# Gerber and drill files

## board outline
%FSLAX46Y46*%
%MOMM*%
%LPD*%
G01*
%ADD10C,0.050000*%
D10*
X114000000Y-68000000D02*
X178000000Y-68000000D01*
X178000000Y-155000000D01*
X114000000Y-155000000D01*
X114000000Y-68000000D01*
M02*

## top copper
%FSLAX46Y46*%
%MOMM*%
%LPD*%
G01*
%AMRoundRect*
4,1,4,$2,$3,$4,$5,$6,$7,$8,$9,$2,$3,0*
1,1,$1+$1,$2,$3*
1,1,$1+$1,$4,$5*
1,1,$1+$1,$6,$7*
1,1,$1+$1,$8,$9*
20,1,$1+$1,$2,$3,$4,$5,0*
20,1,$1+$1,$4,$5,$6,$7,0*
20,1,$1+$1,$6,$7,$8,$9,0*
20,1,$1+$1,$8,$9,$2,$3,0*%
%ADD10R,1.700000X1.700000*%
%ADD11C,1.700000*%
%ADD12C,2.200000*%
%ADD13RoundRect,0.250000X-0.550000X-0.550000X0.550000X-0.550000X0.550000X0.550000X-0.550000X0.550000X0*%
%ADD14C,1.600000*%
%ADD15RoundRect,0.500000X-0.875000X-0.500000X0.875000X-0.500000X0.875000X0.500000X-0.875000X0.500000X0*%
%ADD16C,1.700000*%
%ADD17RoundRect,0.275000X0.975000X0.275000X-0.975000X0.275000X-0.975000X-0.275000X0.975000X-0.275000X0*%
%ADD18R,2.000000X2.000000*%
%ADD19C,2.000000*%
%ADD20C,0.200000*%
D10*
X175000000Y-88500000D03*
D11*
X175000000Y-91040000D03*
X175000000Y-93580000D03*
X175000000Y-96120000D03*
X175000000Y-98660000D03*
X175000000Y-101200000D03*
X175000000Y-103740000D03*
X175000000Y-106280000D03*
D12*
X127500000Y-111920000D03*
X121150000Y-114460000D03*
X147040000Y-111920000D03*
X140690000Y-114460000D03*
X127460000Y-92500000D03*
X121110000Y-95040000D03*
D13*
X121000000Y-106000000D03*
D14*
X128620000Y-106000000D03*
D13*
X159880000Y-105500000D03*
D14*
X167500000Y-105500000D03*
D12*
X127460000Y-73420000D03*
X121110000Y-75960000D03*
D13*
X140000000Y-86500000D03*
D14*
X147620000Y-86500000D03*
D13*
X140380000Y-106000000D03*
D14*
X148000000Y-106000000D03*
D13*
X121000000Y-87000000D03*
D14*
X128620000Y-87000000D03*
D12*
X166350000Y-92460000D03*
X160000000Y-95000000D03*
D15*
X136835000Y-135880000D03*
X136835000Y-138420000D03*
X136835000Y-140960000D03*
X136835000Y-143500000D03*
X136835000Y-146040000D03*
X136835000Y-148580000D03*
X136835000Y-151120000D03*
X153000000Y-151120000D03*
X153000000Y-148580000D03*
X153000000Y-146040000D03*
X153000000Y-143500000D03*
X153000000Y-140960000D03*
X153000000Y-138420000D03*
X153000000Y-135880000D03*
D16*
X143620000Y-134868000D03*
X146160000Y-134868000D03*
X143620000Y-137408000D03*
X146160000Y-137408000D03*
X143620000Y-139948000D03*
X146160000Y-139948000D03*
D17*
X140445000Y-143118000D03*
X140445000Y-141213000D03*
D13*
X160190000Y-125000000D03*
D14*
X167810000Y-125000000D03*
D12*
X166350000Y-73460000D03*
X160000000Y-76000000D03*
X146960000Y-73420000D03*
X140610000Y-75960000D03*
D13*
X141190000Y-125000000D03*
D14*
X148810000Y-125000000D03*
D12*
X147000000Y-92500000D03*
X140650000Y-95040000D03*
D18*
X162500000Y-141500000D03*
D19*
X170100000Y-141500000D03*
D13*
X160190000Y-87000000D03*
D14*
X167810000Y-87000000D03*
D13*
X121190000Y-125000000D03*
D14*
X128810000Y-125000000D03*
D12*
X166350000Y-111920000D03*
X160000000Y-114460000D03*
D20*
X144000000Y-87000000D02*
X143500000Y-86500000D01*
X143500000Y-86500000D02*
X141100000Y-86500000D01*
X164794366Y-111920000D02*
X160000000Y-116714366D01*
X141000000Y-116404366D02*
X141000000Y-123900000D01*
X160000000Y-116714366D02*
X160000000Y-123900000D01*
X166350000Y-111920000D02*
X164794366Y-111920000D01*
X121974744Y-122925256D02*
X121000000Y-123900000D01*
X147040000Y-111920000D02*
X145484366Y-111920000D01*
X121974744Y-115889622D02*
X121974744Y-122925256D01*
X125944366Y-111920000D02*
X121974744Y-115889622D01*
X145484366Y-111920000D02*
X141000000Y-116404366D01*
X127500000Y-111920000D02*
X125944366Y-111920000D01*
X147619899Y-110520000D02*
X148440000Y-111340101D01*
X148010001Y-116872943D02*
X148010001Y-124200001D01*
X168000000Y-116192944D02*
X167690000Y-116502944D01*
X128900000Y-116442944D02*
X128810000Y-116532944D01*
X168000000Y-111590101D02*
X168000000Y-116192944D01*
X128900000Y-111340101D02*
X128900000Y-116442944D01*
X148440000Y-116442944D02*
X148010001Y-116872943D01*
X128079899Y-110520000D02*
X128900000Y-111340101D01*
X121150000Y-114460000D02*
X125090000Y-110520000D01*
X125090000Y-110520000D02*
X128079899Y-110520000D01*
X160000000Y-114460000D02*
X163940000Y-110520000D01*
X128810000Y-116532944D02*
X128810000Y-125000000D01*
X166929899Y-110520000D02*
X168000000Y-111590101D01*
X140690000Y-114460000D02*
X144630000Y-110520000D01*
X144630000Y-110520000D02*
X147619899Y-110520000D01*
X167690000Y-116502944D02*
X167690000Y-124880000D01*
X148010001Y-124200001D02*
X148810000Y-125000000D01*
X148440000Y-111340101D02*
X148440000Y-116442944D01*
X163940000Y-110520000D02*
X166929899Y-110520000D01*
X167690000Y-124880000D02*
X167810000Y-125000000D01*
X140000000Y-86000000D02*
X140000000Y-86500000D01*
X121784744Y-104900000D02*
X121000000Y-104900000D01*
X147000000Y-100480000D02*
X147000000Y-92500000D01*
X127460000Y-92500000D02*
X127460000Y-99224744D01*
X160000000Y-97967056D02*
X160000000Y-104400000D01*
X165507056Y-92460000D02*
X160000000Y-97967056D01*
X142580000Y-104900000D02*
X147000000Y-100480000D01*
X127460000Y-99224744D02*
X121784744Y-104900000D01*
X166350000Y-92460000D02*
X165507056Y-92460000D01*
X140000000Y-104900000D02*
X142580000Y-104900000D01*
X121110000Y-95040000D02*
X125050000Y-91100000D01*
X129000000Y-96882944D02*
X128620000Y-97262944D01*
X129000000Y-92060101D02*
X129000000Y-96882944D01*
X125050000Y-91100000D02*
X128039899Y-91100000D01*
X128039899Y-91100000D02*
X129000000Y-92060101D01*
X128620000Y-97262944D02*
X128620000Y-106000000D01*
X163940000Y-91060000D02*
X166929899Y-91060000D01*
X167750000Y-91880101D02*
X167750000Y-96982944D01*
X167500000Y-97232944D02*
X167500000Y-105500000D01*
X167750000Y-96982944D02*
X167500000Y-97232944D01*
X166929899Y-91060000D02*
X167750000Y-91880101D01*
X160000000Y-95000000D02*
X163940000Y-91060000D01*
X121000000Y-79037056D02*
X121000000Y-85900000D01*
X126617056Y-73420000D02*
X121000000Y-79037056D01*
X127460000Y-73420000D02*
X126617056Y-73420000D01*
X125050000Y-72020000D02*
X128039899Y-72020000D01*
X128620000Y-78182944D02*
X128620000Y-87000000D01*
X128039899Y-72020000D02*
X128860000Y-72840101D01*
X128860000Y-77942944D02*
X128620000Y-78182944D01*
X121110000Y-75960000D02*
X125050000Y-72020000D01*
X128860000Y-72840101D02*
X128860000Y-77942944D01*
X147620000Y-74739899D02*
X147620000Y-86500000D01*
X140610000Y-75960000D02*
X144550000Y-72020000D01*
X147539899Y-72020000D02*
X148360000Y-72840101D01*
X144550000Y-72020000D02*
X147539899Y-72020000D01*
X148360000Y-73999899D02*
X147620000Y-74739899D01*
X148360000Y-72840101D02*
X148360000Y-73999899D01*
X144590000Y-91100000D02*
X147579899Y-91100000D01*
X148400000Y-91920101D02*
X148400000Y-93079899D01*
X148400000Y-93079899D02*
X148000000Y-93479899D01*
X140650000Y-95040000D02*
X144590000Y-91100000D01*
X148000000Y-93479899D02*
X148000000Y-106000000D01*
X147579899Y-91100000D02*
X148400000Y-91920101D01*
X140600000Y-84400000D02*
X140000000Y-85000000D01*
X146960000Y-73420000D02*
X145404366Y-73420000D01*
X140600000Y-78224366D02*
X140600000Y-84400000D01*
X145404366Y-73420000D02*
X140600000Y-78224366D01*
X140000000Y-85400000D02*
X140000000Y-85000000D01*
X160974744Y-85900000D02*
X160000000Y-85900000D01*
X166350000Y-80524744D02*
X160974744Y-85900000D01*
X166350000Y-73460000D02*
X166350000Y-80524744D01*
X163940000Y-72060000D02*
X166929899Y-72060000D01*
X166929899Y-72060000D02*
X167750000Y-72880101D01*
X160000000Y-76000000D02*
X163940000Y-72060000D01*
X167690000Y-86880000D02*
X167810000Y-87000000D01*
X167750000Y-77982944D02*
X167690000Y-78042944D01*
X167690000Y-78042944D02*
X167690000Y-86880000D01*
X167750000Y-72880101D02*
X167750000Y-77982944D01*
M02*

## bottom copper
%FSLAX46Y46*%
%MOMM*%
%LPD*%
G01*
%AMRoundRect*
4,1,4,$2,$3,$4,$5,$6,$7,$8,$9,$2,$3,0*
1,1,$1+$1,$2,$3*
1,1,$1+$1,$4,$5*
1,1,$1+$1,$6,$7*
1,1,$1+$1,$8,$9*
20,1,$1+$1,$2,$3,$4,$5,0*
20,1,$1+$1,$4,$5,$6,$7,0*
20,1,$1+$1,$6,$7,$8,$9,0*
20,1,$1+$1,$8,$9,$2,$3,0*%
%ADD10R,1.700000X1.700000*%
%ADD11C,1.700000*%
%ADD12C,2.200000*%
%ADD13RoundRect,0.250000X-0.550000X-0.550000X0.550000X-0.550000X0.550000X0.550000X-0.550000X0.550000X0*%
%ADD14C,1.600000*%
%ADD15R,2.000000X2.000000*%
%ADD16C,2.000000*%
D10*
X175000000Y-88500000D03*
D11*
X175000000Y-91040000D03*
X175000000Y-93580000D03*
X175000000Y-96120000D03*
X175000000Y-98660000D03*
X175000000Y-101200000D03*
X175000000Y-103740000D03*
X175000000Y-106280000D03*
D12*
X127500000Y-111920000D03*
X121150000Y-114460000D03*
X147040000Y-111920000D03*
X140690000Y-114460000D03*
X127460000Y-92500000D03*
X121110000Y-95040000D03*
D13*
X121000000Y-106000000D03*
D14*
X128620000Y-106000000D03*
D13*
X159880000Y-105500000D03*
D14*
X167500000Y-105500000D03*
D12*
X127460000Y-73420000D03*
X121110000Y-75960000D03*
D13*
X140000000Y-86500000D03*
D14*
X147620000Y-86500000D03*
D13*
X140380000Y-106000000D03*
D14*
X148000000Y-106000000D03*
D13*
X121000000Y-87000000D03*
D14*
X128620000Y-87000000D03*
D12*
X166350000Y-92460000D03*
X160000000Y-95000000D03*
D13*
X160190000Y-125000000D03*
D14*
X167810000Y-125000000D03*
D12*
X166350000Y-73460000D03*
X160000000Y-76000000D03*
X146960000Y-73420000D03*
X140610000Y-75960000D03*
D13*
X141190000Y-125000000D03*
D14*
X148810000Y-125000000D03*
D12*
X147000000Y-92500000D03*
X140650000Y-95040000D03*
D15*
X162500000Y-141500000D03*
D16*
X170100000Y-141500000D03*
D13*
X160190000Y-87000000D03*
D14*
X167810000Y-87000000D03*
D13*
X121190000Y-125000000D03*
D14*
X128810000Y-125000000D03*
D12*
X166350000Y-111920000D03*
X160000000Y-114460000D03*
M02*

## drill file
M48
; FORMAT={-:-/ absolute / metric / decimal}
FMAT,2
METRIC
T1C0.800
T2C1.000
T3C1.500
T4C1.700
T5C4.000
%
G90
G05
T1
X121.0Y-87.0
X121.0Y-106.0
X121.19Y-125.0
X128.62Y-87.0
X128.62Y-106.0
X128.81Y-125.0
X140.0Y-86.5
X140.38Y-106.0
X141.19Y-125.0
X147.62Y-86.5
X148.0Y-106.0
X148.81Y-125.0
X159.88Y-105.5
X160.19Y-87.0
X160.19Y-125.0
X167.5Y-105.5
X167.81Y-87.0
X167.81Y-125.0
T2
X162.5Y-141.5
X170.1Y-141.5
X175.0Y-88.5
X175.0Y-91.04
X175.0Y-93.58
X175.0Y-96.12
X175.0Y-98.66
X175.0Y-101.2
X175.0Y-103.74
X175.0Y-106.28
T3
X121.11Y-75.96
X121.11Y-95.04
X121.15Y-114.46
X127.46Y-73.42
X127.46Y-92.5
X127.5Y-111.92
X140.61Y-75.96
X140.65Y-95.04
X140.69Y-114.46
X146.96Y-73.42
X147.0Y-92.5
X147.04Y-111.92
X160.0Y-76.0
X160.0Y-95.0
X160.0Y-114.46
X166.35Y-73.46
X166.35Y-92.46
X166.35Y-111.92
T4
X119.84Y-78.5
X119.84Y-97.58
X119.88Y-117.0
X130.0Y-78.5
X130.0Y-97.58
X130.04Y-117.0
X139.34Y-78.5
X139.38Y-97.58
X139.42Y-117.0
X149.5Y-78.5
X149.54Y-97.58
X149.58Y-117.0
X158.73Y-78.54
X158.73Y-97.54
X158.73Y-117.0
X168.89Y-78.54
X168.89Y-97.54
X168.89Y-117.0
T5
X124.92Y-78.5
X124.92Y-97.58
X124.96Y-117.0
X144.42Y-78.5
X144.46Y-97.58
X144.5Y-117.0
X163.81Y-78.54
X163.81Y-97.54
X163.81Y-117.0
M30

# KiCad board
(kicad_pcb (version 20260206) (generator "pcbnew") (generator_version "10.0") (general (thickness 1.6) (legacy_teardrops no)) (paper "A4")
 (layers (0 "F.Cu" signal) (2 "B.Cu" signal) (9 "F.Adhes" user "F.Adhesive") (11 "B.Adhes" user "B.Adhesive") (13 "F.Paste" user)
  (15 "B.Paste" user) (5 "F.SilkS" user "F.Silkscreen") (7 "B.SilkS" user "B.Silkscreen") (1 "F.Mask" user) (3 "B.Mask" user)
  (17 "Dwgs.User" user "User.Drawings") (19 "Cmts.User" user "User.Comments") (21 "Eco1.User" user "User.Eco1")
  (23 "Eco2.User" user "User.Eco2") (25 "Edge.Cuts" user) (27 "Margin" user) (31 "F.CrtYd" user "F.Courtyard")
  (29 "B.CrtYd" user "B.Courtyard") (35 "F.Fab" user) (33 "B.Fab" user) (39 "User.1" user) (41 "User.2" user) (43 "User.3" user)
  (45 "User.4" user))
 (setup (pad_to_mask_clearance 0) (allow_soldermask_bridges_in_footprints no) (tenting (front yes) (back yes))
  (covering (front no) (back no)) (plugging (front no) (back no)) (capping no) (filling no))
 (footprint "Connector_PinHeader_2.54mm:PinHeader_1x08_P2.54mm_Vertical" (layer "F.Cu") (at 175 88.5)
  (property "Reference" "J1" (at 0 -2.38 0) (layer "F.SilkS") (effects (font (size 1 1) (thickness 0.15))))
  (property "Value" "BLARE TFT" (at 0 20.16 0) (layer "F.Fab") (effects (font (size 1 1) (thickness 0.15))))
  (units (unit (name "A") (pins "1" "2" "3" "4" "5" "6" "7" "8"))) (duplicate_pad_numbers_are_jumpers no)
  (pad "1" thru_hole rect (at 0 0) (size 1.7 1.7) (drill 1) (layers "*.Cu" "*.Mask") (remove_unused_layers no) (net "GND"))
  (pad "2" thru_hole circle (at 0 2.54) (size 1.7 1.7) (drill 1) (layers "*.Cu" "*.Mask") (remove_unused_layers no) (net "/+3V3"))
  (pad "3" thru_hole circle (at 0 5.08) (size 1.7 1.7) (drill 1) (layers "*.Cu" "*.Mask") (remove_unused_layers no) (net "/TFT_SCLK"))
  (pad "4" thru_hole circle (at 0 7.62) (size 1.7 1.7) (drill 1) (layers "*.Cu" "*.Mask") (remove_unused_layers no) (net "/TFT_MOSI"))
  (pad "5" thru_hole circle (at 0 10.16) (size 1.7 1.7) (drill 1) (layers "*.Cu" "*.Mask") (remove_unused_layers no) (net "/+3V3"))
  (pad "6" thru_hole circle (at 0 12.7) (size 1.7 1.7) (drill 1) (layers "*.Cu" "*.Mask") (remove_unused_layers no) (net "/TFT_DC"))
  (pad "7" thru_hole circle (at 0 15.24) (size 1.7 1.7) (drill 1) (layers "*.Cu" "*.Mask") (remove_unused_layers no) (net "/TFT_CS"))
  (pad "8" thru_hole circle (at 0 17.78) (size 1.7 1.7) (drill 1) (layers "*.Cu" "*.Mask") (remove_unused_layers no) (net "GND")))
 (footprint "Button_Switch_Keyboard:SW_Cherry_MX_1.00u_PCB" (layer "F.Cu") (at 127.5 111.92)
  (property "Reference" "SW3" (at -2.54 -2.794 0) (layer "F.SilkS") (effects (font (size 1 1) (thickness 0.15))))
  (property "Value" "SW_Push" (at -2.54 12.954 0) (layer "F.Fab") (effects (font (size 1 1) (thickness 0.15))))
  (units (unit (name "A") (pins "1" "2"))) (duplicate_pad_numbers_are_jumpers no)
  (pad "" np_thru_hole circle (at -7.62 5.08) (size 1.7 1.7) (drill 1.7) (layers "*.Cu" "*.Mask"))
  (pad "" np_thru_hole circle (at -2.54 5.08) (size 4 4) (drill 4) (layers "*.Cu" "*.Mask"))
  (pad "" np_thru_hole circle (at 2.54 5.08) (size 1.7 1.7) (drill 1.7) (layers "*.Cu" "*.Mask"))
  (pad "1" thru_hole circle (at 0 0) (size 2.2 2.2) (drill 1.5) (layers "*.Cu" "*.Mask") (remove_unused_layers no) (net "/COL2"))
  (pad "2" thru_hole circle (at -6.35 2.54) (size 2.2 2.2) (drill 1.5) (layers "*.Cu" "*.Mask") (remove_unused_layers no) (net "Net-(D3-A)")))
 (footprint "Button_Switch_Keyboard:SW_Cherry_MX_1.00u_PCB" (layer "F.Cu") (at 147.04 111.92)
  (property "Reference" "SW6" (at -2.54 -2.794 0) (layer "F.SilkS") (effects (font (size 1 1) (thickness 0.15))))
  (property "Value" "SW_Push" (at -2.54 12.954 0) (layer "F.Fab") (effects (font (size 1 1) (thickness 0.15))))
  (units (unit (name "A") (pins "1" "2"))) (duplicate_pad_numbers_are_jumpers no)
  (pad "" np_thru_hole circle (at -7.62 5.08) (size 1.7 1.7) (drill 1.7) (layers "*.Cu" "*.Mask"))
  (pad "" np_thru_hole circle (at -2.54 5.08) (size 4 4) (drill 4) (layers "*.Cu" "*.Mask"))
  (pad "" np_thru_hole circle (at 2.54 5.08) (size 1.7 1.7) (drill 1.7) (layers "*.Cu" "*.Mask"))
  (pad "1" thru_hole circle (at 0 0) (size 2.2 2.2) (drill 1.5) (layers "*.Cu" "*.Mask") (remove_unused_layers no) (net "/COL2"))
  (pad "2" thru_hole circle (at -6.35 2.54) (size 2.2 2.2) (drill 1.5) (layers "*.Cu" "*.Mask") (remove_unused_layers no) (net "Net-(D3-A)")))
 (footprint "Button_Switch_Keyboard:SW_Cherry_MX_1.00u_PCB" (layer "F.Cu") (at 127.46 92.5)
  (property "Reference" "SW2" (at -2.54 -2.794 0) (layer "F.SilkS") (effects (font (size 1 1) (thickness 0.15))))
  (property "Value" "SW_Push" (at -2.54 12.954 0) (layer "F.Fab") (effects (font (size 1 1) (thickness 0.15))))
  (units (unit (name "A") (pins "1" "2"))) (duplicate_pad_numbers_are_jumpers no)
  (pad "" np_thru_hole circle (at -7.62 5.08) (size 1.7 1.7) (drill 1.7) (layers "*.Cu" "*.Mask"))
  (pad "" np_thru_hole circle (at -2.54 5.08) (size 4 4) (drill 4) (layers "*.Cu" "*.Mask"))
  (pad "" np_thru_hole circle (at 2.54 5.08) (size 1.7 1.7) (drill 1.7) (layers "*.Cu" "*.Mask"))
  (pad "1" thru_hole circle (at 0 0) (size 2.2 2.2) (drill 1.5) (layers "*.Cu" "*.Mask") (remove_unused_layers no) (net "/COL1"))
  (pad "2" thru_hole circle (at -6.35 2.54) (size 2.2 2.2) (drill 1.5) (layers "*.Cu" "*.Mask") (remove_unused_layers no) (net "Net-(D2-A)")))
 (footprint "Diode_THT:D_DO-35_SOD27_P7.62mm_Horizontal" (layer "F.Cu") (at 121 106)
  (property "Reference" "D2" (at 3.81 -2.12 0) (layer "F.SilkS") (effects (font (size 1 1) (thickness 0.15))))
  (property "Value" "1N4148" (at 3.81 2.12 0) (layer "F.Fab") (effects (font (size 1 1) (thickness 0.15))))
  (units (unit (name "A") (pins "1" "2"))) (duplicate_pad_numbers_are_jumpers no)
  (pad "1" thru_hole roundrect (at 0 0) (size 1.6 1.6) (drill 0.8) (layers "*.Cu" "*.Mask") (remove_unused_layers no)
   (roundrect_rratio 0.15625) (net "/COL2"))
  (pad "2" thru_hole circle (at 7.62 0) (size 1.6 1.6) (drill 0.8) (layers "*.Cu" "*.Mask") (remove_unused_layers no) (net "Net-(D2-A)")))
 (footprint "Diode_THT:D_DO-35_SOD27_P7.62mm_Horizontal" (layer "F.Cu") (at 159.88 105.5)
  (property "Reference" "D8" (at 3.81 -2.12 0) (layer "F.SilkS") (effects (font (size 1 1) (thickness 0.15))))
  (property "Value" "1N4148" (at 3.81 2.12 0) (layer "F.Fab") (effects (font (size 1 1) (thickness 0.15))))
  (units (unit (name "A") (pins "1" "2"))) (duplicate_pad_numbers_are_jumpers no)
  (pad "1" thru_hole roundrect (at 0 0) (size 1.6 1.6) (drill 0.8) (layers "*.Cu" "*.Mask") (remove_unused_layers no)
   (roundrect_rratio 0.15625) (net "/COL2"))
  (pad "2" thru_hole circle (at 7.62 0) (size 1.6 1.6) (drill 0.8) (layers "*.Cu" "*.Mask") (remove_unused_layers no) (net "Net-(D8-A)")))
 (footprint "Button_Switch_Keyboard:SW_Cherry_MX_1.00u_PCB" (layer "F.Cu") (at 127.46 73.42)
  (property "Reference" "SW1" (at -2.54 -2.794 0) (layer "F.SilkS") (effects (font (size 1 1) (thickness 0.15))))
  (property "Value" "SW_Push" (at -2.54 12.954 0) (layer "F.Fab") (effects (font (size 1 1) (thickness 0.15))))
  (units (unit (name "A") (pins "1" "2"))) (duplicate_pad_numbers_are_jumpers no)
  (pad "" np_thru_hole circle (at -7.62 5.08) (size 1.7 1.7) (drill 1.7) (layers "*.Cu" "*.Mask"))
  (pad "" np_thru_hole circle (at -2.54 5.08) (size 4 4) (drill 4) (layers "*.Cu" "*.Mask"))
  (pad "" np_thru_hole circle (at 2.54 5.08) (size 1.7 1.7) (drill 1.7) (layers "*.Cu" "*.Mask"))
  (pad "1" thru_hole circle (at 0 0) (size 2.2 2.2) (drill 1.5) (layers "*.Cu" "*.Mask") (remove_unused_layers no) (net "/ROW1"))
  (pad "2" thru_hole circle (at -6.35 2.54) (size 2.2 2.2) (drill 1.5) (layers "*.Cu" "*.Mask") (remove_unused_layers no) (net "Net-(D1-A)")))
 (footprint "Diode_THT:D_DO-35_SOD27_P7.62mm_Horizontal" (layer "F.Cu") (at 140 86.5)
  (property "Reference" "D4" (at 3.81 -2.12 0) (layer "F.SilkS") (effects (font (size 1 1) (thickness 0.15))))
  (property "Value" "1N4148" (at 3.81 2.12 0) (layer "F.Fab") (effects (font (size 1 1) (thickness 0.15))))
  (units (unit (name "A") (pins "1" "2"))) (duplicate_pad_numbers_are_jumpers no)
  (pad "1" thru_hole roundrect (at 0 0) (size 1.6 1.6) (drill 0.8) (layers "*.Cu" "*.Mask") (remove_unused_layers no)
   (roundrect_rratio 0.15625) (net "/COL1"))
  (pad "2" thru_hole circle (at 7.62 0) (size 1.6 1.6) (drill 0.8) (layers "*.Cu" "*.Mask") (remove_unused_layers no) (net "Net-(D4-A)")))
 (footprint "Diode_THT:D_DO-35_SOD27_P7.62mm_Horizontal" (layer "F.Cu") (at 140.38 106)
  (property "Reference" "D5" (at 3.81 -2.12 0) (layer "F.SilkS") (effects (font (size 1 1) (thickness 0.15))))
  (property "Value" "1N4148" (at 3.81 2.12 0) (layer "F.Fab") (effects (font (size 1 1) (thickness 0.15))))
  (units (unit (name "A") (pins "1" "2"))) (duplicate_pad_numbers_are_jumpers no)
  (pad "1" thru_hole roundrect (at 0 0) (size 1.6 1.6) (drill 0.8) (layers "*.Cu" "*.Mask") (remove_unused_layers no)
   (roundrect_rratio 0.15625) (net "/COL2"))
  (pad "2" thru_hole circle (at 7.62 0) (size 1.6 1.6) (drill 0.8) (layers "*.Cu" "*.Mask") (remove_unused_layers no) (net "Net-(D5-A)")))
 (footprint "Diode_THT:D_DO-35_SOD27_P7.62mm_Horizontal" (layer "F.Cu") (at 121 87)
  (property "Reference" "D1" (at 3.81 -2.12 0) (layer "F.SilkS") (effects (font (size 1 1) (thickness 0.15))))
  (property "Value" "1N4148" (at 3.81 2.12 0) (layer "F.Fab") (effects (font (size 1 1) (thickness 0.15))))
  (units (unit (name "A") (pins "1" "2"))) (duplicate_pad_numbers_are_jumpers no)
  (pad "1" thru_hole roundrect (at 0 0) (size 1.6 1.6) (drill 0.8) (layers "*.Cu" "*.Mask") (remove_unused_layers no)
   (roundrect_rratio 0.15625) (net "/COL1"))
  (pad "2" thru_hole circle (at 7.62 0) (size 1.6 1.6) (drill 0.8) (layers "*.Cu" "*.Mask") (remove_unused_layers no) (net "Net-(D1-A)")))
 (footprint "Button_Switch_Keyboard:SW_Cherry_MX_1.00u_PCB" (layer "F.Cu") (at 166.35 92.46)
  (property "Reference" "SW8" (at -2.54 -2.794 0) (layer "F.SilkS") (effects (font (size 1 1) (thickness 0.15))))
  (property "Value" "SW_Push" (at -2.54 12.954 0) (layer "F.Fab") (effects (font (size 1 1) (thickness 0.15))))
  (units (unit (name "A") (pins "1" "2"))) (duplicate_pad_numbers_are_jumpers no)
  (pad "" np_thru_hole circle (at -7.62 5.08) (size 1.7 1.7) (drill 1.7) (layers "*.Cu" "*.Mask"))
  (pad "" np_thru_hole circle (at -2.54 5.08) (size 4 4) (drill 4) (layers "*.Cu" "*.Mask"))
  (pad "" np_thru_hole circle (at 2.54 5.08) (size 1.7 1.7) (drill 1.7) (layers "*.Cu" "*.Mask"))
  (pad "1" thru_hole circle (at 0 0) (size 2.2 2.2) (drill 1.5) (layers "*.Cu" "*.Mask") (remove_unused_layers no) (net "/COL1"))
  (pad "2" thru_hole circle (at -6.35 2.54) (size 2.2 2.2) (drill 1.5) (layers "*.Cu" "*.Mask") (remove_unused_layers no) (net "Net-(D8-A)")))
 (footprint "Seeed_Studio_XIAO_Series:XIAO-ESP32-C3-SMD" (layer "F.Cu") (at 136 154)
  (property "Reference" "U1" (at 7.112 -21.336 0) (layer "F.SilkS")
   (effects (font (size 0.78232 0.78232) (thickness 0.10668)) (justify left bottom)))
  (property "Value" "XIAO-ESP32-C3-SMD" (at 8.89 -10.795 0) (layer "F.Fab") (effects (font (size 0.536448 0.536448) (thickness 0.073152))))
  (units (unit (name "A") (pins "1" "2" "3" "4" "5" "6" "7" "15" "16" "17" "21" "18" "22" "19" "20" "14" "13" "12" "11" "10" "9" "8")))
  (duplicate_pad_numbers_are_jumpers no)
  (pad "1" smd roundrect (at 0.835 -18.12) (size 2.75 2) (layers "F.Cu" "F.Mask" "F.Paste") (roundrect_rratio 0.25) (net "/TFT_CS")
   (solder_mask_margin 0.0508) (thermal_bridge_angle 45))
  (pad "2" smd roundrect (at 0.835 -15.58) (size 2.75 2) (layers "F.Cu" "F.Mask" "F.Paste") (roundrect_rratio 0.25) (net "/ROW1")
   (solder_mask_margin 0.0508) (thermal_bridge_angle 45))
  (pad "3" smd roundrect (at 0.835 -13.04) (size 2.75 2) (layers "F.Cu" "F.Mask" "F.Paste") (roundrect_rratio 0.25) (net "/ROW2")
   (solder_mask_margin 0.0508) (thermal_bridge_angle 45))
  (pad "4" smd roundrect (at 0.835 -10.5) (size 2.75 2) (layers "F.Cu" "F.Mask" "F.Paste") (roundrect_rratio 0.25) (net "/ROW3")
   (solder_mask_margin 0.0508) (thermal_bridge_angle 45))
  (pad "5" smd roundrect (at 0.835 -7.96) (size 2.75 2) (layers "F.Cu" "F.Mask" "F.Paste") (roundrect_rratio 0.25) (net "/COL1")
   (solder_mask_margin 0.0508) (thermal_bridge_angle 45))
  (pad "6" smd roundrect (at 0.835 -5.42) (size 2.75 2) (layers "F.Cu" "F.Mask" "F.Paste") (roundrect_rratio 0.25) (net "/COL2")
   (solder_mask_margin 0.0508) (thermal_bridge_angle 45))
  (pad "7" smd roundrect (at 0.835 -2.88) (size 2.75 2) (layers "F.Cu" "F.Mask" "F.Paste") (roundrect_rratio 0.25) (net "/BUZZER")
   (solder_mask_margin 0.0508) (thermal_bridge_angle 45))
  (pad "8" smd roundrect (at 17 -2.88) (size 2.75 2) (layers "F.Cu" "F.Mask" "F.Paste") (roundrect_rratio 0.25) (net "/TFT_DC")
   (solder_mask_margin 0.0508) (thermal_bridge_angle 45))
  (pad "9" smd roundrect (at 17 -5.42) (size 2.75 2) (layers "F.Cu" "F.Mask" "F.Paste") (roundrect_rratio 0.25) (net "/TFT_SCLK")
   (solder_mask_margin 0.0508) (thermal_bridge_angle 45))
  (pad "10" smd roundrect (at 17 -7.96) (size 2.75 2) (layers "F.Cu" "F.Mask" "F.Paste") (roundrect_rratio 0.25) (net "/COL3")
   (solder_mask_margin 0.0508) (thermal_bridge_angle 45))
  (pad "11" smd roundrect (at 17 -10.5) (size 2.75 2) (layers "F.Cu" "F.Mask" "F.Paste") (roundrect_rratio 0.25) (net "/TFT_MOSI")
   (solder_mask_margin 0.0508) (thermal_bridge_angle 45))
  (pad "12" smd roundrect (at 17 -13.04) (size 2.75 2) (layers "F.Cu" "F.Mask" "F.Paste") (roundrect_rratio 0.25) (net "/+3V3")
   (solder_mask_margin 0.0508) (thermal_bridge_angle 45))
  (pad "13" smd roundrect (at 17 -15.58) (size 2.75 2) (layers "F.Cu" "F.Mask" "F.Paste") (roundrect_rratio 0.25) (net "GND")
   (solder_mask_margin 0.0508) (thermal_bridge_angle 45))
  (pad "14" smd roundrect (at 17 -18.12) (size 2.75 2) (layers "F.Cu" "F.Mask" "F.Paste") (roundrect_rratio 0.25)
   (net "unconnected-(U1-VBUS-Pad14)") (solder_mask_margin 0.0508) (thermal_bridge_angle 45))
  (pad "15" smd circle (at 7.62 -19.132) (size 1.7 1.7) (layers "F.Cu" "F.Mask" "F.Paste") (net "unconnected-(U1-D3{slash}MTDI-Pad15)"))
  (pad "16" smd circle (at 10.16 -19.132) (size 1.7 1.7) (layers "F.Cu" "F.Mask" "F.Paste") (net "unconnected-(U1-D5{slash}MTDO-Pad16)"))
  (pad "17" smd circle (at 7.62 -16.592) (size 1.7 1.7) (layers "F.Cu" "F.Mask" "F.Paste") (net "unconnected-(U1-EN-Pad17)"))
  (pad "18" smd circle (at 10.16 -16.592) (size 1.7 1.7) (layers "F.Cu" "F.Mask" "F.Paste") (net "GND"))
  (pad "19" smd circle (at 7.62 -14.052) (size 1.7 1.7) (layers "F.Cu" "F.Mask" "F.Paste") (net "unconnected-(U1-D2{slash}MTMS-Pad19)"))
  (pad "20" smd circle (at 10.16 -14.052) (size 1.7 1.7) (layers "F.Cu" "F.Mask" "F.Paste") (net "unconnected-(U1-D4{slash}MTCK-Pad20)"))
  (pad "21" smd roundrect (at 4.445 -10.882 180) (size 2.5 1.1) (layers "F.Cu" "F.Mask" "F.Paste") (roundrect_rratio 0.25)
   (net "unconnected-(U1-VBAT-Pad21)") (thermal_bridge_angle 45))
  (pad "22" smd roundrect (at 4.445 -12.787 180) (size 2.5 1.1) (layers "F.Cu" "F.Mask" "F.Paste") (roundrect_rratio 0.25) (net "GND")
   (thermal_bridge_angle 45)))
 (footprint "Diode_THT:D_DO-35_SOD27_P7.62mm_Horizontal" (layer "F.Cu") (at 160.19 125)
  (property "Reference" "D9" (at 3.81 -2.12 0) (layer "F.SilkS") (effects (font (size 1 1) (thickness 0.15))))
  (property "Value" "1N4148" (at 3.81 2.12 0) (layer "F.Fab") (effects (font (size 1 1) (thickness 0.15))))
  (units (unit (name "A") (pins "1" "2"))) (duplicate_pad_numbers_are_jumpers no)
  (pad "1" thru_hole roundrect (at 0 0) (size 1.6 1.6) (drill 0.8) (layers "*.Cu" "*.Mask") (remove_unused_layers no)
   (roundrect_rratio 0.15625) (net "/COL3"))
  (pad "2" thru_hole circle (at 7.62 0) (size 1.6 1.6) (drill 0.8) (layers "*.Cu" "*.Mask") (remove_unused_layers no) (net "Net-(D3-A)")))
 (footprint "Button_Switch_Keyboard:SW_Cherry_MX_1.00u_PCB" (layer "F.Cu") (at 166.35 73.46)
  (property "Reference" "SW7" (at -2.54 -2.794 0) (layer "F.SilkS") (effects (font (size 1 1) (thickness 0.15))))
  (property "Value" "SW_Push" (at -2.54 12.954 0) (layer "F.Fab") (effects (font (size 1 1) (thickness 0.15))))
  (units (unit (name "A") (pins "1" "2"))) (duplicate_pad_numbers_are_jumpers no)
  (pad "" np_thru_hole circle (at -7.62 5.08) (size 1.7 1.7) (drill 1.7) (layers "*.Cu" "*.Mask"))
  (pad "" np_thru_hole circle (at -2.54 5.08) (size 4 4) (drill 4) (layers "*.Cu" "*.Mask"))
  (pad "" np_thru_hole circle (at 2.54 5.08) (size 1.7 1.7) (drill 1.7) (layers "*.Cu" "*.Mask"))
  (pad "1" thru_hole circle (at 0 0) (size 2.2 2.2) (drill 1.5) (layers "*.Cu" "*.Mask") (remove_unused_layers no) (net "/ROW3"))
  (pad "2" thru_hole circle (at -6.35 2.54) (size 2.2 2.2) (drill 1.5) (layers "*.Cu" "*.Mask") (remove_unused_layers no) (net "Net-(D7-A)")))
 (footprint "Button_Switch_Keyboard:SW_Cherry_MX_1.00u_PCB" (layer "F.Cu") (at 146.96 73.42)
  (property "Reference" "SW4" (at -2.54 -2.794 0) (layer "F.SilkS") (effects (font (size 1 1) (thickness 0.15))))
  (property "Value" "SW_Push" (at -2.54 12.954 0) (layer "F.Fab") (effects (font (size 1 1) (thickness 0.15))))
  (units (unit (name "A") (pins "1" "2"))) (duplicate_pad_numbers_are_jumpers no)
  (pad "" np_thru_hole circle (at -7.62 5.08) (size 1.7 1.7) (drill 1.7) (layers "*.Cu" "*.Mask"))
  (pad "" np_thru_hole circle (at -2.54 5.08) (size 4 4) (drill 4) (layers "*.Cu" "*.Mask"))
  (pad "" np_thru_hole circle (at 2.54 5.08) (size 1.7 1.7) (drill 1.7) (layers "*.Cu" "*.Mask"))
  (pad "1" thru_hole circle (at 0 0) (size 2.2 2.2) (drill 1.5) (layers "*.Cu" "*.Mask") (remove_unused_layers no) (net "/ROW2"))
  (pad "2" thru_hole circle (at -6.35 2.54) (size 2.2 2.2) (drill 1.5) (layers "*.Cu" "*.Mask") (remove_unused_layers no) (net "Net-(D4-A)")))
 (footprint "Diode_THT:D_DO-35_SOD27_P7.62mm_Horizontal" (layer "F.Cu") (at 141.19 125)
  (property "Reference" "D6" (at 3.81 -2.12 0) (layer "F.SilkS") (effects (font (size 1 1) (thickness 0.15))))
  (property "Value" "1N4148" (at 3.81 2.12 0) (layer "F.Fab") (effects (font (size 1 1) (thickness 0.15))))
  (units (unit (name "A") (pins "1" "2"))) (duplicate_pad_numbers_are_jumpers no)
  (pad "1" thru_hole roundrect (at 0 0) (size 1.6 1.6) (drill 0.8) (layers "*.Cu" "*.Mask") (remove_unused_layers no)
   (roundrect_rratio 0.15625) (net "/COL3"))
  (pad "2" thru_hole circle (at 7.62 0) (size 1.6 1.6) (drill 0.8) (layers "*.Cu" "*.Mask") (remove_unused_layers no) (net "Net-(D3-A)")))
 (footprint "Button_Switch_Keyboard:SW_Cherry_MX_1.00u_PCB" (layer "F.Cu") (at 147 92.5)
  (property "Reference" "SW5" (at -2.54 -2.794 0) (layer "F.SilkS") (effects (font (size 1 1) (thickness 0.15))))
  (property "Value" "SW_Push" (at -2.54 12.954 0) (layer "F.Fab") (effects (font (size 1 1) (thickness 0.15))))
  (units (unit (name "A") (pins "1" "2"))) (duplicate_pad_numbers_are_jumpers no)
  (pad "" np_thru_hole circle (at -7.62 5.08) (size 1.7 1.7) (drill 1.7) (layers "*.Cu" "*.Mask"))
  (pad "" np_thru_hole circle (at -2.54 5.08) (size 4 4) (drill 4) (layers "*.Cu" "*.Mask"))
  (pad "" np_thru_hole circle (at 2.54 5.08) (size 1.7 1.7) (drill 1.7) (layers "*.Cu" "*.Mask"))
  (pad "1" thru_hole circle (at 0 0) (size 2.2 2.2) (drill 1.5) (layers "*.Cu" "*.Mask") (remove_unused_layers no) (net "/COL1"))
  (pad "2" thru_hole circle (at -6.35 2.54) (size 2.2 2.2) (drill 1.5) (layers "*.Cu" "*.Mask") (remove_unused_layers no) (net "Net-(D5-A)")))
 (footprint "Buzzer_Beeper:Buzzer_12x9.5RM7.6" (layer "F.Cu") (at 162.5 141.5)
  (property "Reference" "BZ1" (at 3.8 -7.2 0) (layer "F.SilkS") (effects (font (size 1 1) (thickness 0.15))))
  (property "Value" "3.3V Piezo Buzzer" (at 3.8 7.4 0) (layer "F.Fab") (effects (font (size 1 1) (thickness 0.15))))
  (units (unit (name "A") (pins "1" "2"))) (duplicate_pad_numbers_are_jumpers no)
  (pad "1" thru_hole rect (at 0 0) (size 2 2) (drill 1) (layers "*.Cu" "*.Mask") (remove_unused_layers no) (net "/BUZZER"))
  (pad "2" thru_hole circle (at 7.6 0) (size 2 2) (drill 1) (layers "*.Cu" "*.Mask") (remove_unused_layers no) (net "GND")))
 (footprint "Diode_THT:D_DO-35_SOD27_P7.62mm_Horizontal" (layer "F.Cu") (at 160.19 87)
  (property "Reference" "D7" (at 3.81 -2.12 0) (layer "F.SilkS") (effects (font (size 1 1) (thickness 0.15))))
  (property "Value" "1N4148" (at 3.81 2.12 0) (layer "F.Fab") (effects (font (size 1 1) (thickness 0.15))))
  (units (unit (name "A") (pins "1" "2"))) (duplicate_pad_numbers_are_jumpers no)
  (pad "1" thru_hole roundrect (at 0 0) (size 1.6 1.6) (drill 0.8) (layers "*.Cu" "*.Mask") (remove_unused_layers no)
   (roundrect_rratio 0.15625) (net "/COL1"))
  (pad "2" thru_hole circle (at 7.62 0) (size 1.6 1.6) (drill 0.8) (layers "*.Cu" "*.Mask") (remove_unused_layers no) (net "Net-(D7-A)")))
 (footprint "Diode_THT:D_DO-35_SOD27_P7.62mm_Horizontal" (layer "F.Cu") (at 121.19 125)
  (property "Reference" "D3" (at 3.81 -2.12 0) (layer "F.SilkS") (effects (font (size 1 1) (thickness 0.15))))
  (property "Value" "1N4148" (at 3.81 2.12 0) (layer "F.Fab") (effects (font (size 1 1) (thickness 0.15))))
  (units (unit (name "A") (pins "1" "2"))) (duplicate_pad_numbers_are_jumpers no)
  (pad "1" thru_hole roundrect (at 0 0) (size 1.6 1.6) (drill 0.8) (layers "*.Cu" "*.Mask") (remove_unused_layers no)
   (roundrect_rratio 0.15625) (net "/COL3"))
  (pad "2" thru_hole circle (at 7.62 0) (size 1.6 1.6) (drill 0.8) (layers "*.Cu" "*.Mask") (remove_unused_layers no) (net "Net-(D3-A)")))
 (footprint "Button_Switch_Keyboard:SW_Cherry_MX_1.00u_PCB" (layer "F.Cu") (at 166.35 111.92)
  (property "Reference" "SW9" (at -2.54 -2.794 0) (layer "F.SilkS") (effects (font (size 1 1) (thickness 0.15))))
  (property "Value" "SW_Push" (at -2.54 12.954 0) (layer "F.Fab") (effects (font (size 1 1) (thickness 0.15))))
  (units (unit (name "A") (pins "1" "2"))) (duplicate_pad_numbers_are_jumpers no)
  (pad "" np_thru_hole circle (at -7.62 5.08) (size 1.7 1.7) (drill 1.7) (layers "*.Cu" "*.Mask"))
  (pad "" np_thru_hole circle (at -2.54 5.08) (size 4 4) (drill 4) (layers "*.Cu" "*.Mask"))
  (pad "" np_thru_hole circle (at 2.54 5.08) (size 1.7 1.7) (drill 1.7) (layers "*.Cu" "*.Mask"))
  (pad "1" thru_hole circle (at 0 0) (size 2.2 2.2) (drill 1.5) (layers "*.Cu" "*.Mask") (remove_unused_layers no) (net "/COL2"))
  (pad "2" thru_hole circle (at -6.35 2.54) (size 2.2 2.2) (drill 1.5) (layers "*.Cu" "*.Mask") (remove_unused_layers no) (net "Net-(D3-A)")))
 (gr_rect (start 114 68) (end 178 155) (stroke (width 0.05) (type default)) (fill no) (layer "Edge.Cuts"))
 (segment (start 144 87) (end 143.5 86.5) (width 0.2) (layer "F.Cu") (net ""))
 (segment (start 143.5 86.5) (end 141.1 86.5) (width 0.2) (layer "F.Cu") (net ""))
 (segment (start 164.794366 111.92) (end 160 116.714366) (width 0.2) (layer "F.Cu") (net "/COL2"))
 (segment (start 141 116.404366) (end 141 123.9) (width 0.2) (layer "F.Cu") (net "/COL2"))
 (segment (start 160 116.714366) (end 160 123.9) (width 0.2) (layer "F.Cu") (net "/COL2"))
 (segment (start 166.35 111.92) (end 164.794366 111.92) (width 0.2) (layer "F.Cu") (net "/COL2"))
 (segment (start 121.974744 122.925256) (end 121 123.9) (width 0.2) (layer "F.Cu") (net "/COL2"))
 (segment (start 147.04 111.92) (end 145.484366 111.92) (width 0.2) (layer "F.Cu") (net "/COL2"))
 (segment (start 121.974744 115.889622) (end 121.974744 122.925256) (width 0.2) (layer "F.Cu") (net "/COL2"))
 (segment (start 125.944366 111.92) (end 121.974744 115.889622) (width 0.2) (layer "F.Cu") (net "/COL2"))
 (segment (start 145.484366 111.92) (end 141 116.404366) (width 0.2) (layer "F.Cu") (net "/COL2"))
 (segment (start 127.5 111.92) (end 125.944366 111.92) (width 0.2) (layer "F.Cu") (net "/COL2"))
 (segment (start 147.619899 110.52) (end 148.44 111.340101) (width 0.2) (layer "F.Cu") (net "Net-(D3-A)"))
 (segment (start 148.010001 116.872943) (end 148.010001 124.200001) (width 0.2) (layer "F.Cu") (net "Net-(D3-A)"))
 (segment (start 168 116.192944) (end 167.69 116.502944) (width 0.2) (layer "F.Cu") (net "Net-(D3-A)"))
 (segment (start 128.9 116.442944) (end 128.81 116.532944) (width 0.2) (layer "F.Cu") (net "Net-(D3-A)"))
 (segment (start 168 111.590101) (end 168 116.192944) (width 0.2) (layer "F.Cu") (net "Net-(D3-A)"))
 (segment (start 128.9 111.340101) (end 128.9 116.442944) (width 0.2) (layer "F.Cu") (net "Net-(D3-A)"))
 (segment (start 148.44 116.442944) (end 148.010001 116.872943) (width 0.2) (layer "F.Cu") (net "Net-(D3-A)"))
 (segment (start 128.079899 110.52) (end 128.9 111.340101) (width 0.2) (layer "F.Cu") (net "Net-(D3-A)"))
 (segment (start 121.15 114.46) (end 125.09 110.52) (width 0.2) (layer "F.Cu") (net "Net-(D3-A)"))
 (segment (start 125.09 110.52) (end 128.079899 110.52) (width 0.2) (layer "F.Cu") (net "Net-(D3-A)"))
 (segment (start 160 114.46) (end 163.94 110.52) (width 0.2) (layer "F.Cu") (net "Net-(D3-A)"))
 (segment (start 128.81 116.532944) (end 128.81 125) (width 0.2) (layer "F.Cu") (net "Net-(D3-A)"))
 (segment (start 166.929899 110.52) (end 168 111.590101) (width 0.2) (layer "F.Cu") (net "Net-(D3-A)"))
 (segment (start 140.69 114.46) (end 144.63 110.52) (width 0.2) (layer "F.Cu") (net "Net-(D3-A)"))
 (segment (start 144.63 110.52) (end 147.619899 110.52) (width 0.2) (layer "F.Cu") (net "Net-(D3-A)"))
 (segment (start 167.69 116.502944) (end 167.69 124.88) (width 0.2) (layer "F.Cu") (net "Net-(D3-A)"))
 (segment (start 148.010001 124.200001) (end 148.81 125) (width 0.2) (layer "F.Cu") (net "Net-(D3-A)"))
 (segment (start 148.44 111.340101) (end 148.44 116.442944) (width 0.2) (layer "F.Cu") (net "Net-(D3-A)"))
 (segment (start 163.94 110.52) (end 166.929899 110.52) (width 0.2) (layer "F.Cu") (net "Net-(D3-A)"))
 (segment (start 167.69 124.88) (end 167.81 125) (width 0.2) (layer "F.Cu") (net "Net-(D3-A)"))
 (segment (start 140 86) (end 140 86.5) (width 0.2) (layer "F.Cu") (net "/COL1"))
 (segment (start 121.784744 104.9) (end 121 104.9) (width 0.2) (layer "F.Cu") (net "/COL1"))
 (segment (start 147 100.48) (end 147 92.5) (width 0.2) (layer "F.Cu") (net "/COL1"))
 (segment (start 127.46 92.5) (end 127.46 99.224744) (width 0.2) (layer "F.Cu") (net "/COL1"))
 (segment (start 160 97.967056) (end 160 104.4) (width 0.2) (layer "F.Cu") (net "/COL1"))
 (segment (start 165.507056 92.46) (end 160 97.967056) (width 0.2) (layer "F.Cu") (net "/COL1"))
 (segment (start 142.58 104.9) (end 147 100.48) (width 0.2) (layer "F.Cu") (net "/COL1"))
 (segment (start 127.46 99.224744) (end 121.784744 104.9) (width 0.2) (layer "F.Cu") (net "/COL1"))
 (segment (start 166.35 92.46) (end 165.507056 92.46) (width 0.2) (layer "F.Cu") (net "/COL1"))
 (segment (start 140 104.9) (end 142.58 104.9) (width 0.2) (layer "F.Cu") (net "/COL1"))
 (segment (start 121.11 95.04) (end 125.05 91.1) (width 0.2) (layer "F.Cu") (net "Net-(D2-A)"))
 (segment (start 129 96.882944) (end 128.62 97.262944) (width 0.2) (layer "F.Cu") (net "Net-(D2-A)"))
 (segment (start 129 92.060101) (end 129 96.882944) (width 0.2) (layer "F.Cu") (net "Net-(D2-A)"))
 (segment (start 125.05 91.1) (end 128.039899 91.1) (width 0.2) (layer "F.Cu") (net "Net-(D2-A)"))
 (segment (start 128.039899 91.1) (end 129 92.060101) (width 0.2) (layer "F.Cu") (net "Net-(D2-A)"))
 (segment (start 128.62 97.262944) (end 128.62 106) (width 0.2) (layer "F.Cu") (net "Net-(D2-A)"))
 (segment (start 163.94 91.06) (end 166.929899 91.06) (width 0.2) (layer "F.Cu") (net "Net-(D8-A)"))
 (segment (start 167.75 91.880101) (end 167.75 96.982944) (width 0.2) (layer "F.Cu") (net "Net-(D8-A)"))
 (segment (start 167.5 97.232944) (end 167.5 105.5) (width 0.2) (layer "F.Cu") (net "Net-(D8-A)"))
 (segment (start 167.75 96.982944) (end 167.5 97.232944) (width 0.2) (layer "F.Cu") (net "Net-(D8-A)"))
 (segment (start 166.929899 91.06) (end 167.75 91.880101) (width 0.2) (layer "F.Cu") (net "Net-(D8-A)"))
 (segment (start 160 95) (end 163.94 91.06) (width 0.2) (layer "F.Cu") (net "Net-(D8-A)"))
 (segment (start 121 79.037056) (end 121 85.9) (width 0.2) (layer "F.Cu") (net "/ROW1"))
 (segment (start 126.617056 73.42) (end 121 79.037056) (width 0.2) (layer "F.Cu") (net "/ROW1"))
 (segment (start 127.46 73.42) (end 126.617056 73.42) (width 0.2) (layer "F.Cu") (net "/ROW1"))
 (segment (start 125.05 72.02) (end 128.039899 72.02) (width 0.2) (layer "F.Cu") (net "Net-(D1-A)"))
 (segment (start 128.62 78.182944) (end 128.62 87) (width 0.2) (layer "F.Cu") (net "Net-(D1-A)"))
 (segment (start 128.039899 72.02) (end 128.86 72.840101) (width 0.2) (layer "F.Cu") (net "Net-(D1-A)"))
 (segment (start 128.86 77.942944) (end 128.62 78.182944) (width 0.2) (layer "F.Cu") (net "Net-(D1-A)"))
 (segment (start 121.11 75.96) (end 125.05 72.02) (width 0.2) (layer "F.Cu") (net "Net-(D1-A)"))
 (segment (start 128.86 72.840101) (end 128.86 77.942944) (width 0.2) (layer "F.Cu") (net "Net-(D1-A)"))
 (segment (start 147.62 74.739899) (end 147.62 86.5) (width 0.2) (layer "F.Cu") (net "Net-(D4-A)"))
 (segment (start 140.61 75.96) (end 144.55 72.02) (width 0.2) (layer "F.Cu") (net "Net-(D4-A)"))
 (segment (start 147.539899 72.02) (end 148.36 72.840101) (width 0.2) (layer "F.Cu") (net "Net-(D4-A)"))
 (segment (start 144.55 72.02) (end 147.539899 72.02) (width 0.2) (layer "F.Cu") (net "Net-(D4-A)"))
 (segment (start 148.36 73.999899) (end 147.62 74.739899) (width 0.2) (layer "F.Cu") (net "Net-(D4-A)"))
 (segment (start 148.36 72.840101) (end 148.36 73.999899) (width 0.2) (layer "F.Cu") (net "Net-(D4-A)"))
 (segment (start 144.59 91.1) (end 147.579899 91.1) (width 0.2) (layer "F.Cu") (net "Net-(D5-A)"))
 (segment (start 148.4 91.920101) (end 148.4 93.079899) (width 0.2) (layer "F.Cu") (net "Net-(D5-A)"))
 (segment (start 148.4 93.079899) (end 148 93.479899) (width 0.2) (layer "F.Cu") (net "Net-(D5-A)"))
 (segment (start 140.65 95.04) (end 144.59 91.1) (width 0.2) (layer "F.Cu") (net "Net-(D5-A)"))
 (segment (start 148 93.479899) (end 148 106) (width 0.2) (layer "F.Cu") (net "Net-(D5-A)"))
 (segment (start 147.579899 91.1) (end 148.4 91.920101) (width 0.2) (layer "F.Cu") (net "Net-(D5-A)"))
 (segment (start 140.6 84.4) (end 140 85) (width 0.2) (layer "F.Cu") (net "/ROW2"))
 (segment (start 146.96 73.42) (end 145.404366 73.42) (width 0.2) (layer "F.Cu") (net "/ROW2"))
 (segment (start 140.6 78.224366) (end 140.6 84.4) (width 0.2) (layer "F.Cu") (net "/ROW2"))
 (segment (start 145.404366 73.42) (end 140.6 78.224366) (width 0.2) (layer "F.Cu") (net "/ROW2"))
 (segment (start 140 85.4) (end 140 85) (width 0.2) (layer "F.Cu") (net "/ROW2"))
 (segment (start 160.974744 85.9) (end 160 85.9) (width 0.2) (layer "F.Cu") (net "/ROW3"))
 (segment (start 166.35 80.524744) (end 160.974744 85.9) (width 0.2) (layer "F.Cu") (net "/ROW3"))
 (segment (start 166.35 73.46) (end 166.35 80.524744) (width 0.2) (layer "F.Cu") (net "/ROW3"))
 (segment (start 163.94 72.06) (end 166.929899 72.06) (width 0.2) (layer "F.Cu") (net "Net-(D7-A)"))
 (segment (start 166.929899 72.06) (end 167.75 72.880101) (width 0.2) (layer "F.Cu") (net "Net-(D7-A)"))
 (segment (start 160 76) (end 163.94 72.06) (width 0.2) (layer "F.Cu") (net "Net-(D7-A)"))
 (segment (start 167.69 86.88) (end 167.81 87) (width 0.2) (layer "F.Cu") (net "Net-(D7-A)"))
 (segment (start 167.75 77.982944) (end 167.69 78.042944) (width 0.2) (layer "F.Cu") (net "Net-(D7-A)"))
 (segment (start 167.69 78.042944) (end 167.69 86.88) (width 0.2) (layer "F.Cu") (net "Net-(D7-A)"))
 (segment (start 167.75 72.880101) (end 167.75 77.982944) (width 0.2) (layer "F.Cu") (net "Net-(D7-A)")))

